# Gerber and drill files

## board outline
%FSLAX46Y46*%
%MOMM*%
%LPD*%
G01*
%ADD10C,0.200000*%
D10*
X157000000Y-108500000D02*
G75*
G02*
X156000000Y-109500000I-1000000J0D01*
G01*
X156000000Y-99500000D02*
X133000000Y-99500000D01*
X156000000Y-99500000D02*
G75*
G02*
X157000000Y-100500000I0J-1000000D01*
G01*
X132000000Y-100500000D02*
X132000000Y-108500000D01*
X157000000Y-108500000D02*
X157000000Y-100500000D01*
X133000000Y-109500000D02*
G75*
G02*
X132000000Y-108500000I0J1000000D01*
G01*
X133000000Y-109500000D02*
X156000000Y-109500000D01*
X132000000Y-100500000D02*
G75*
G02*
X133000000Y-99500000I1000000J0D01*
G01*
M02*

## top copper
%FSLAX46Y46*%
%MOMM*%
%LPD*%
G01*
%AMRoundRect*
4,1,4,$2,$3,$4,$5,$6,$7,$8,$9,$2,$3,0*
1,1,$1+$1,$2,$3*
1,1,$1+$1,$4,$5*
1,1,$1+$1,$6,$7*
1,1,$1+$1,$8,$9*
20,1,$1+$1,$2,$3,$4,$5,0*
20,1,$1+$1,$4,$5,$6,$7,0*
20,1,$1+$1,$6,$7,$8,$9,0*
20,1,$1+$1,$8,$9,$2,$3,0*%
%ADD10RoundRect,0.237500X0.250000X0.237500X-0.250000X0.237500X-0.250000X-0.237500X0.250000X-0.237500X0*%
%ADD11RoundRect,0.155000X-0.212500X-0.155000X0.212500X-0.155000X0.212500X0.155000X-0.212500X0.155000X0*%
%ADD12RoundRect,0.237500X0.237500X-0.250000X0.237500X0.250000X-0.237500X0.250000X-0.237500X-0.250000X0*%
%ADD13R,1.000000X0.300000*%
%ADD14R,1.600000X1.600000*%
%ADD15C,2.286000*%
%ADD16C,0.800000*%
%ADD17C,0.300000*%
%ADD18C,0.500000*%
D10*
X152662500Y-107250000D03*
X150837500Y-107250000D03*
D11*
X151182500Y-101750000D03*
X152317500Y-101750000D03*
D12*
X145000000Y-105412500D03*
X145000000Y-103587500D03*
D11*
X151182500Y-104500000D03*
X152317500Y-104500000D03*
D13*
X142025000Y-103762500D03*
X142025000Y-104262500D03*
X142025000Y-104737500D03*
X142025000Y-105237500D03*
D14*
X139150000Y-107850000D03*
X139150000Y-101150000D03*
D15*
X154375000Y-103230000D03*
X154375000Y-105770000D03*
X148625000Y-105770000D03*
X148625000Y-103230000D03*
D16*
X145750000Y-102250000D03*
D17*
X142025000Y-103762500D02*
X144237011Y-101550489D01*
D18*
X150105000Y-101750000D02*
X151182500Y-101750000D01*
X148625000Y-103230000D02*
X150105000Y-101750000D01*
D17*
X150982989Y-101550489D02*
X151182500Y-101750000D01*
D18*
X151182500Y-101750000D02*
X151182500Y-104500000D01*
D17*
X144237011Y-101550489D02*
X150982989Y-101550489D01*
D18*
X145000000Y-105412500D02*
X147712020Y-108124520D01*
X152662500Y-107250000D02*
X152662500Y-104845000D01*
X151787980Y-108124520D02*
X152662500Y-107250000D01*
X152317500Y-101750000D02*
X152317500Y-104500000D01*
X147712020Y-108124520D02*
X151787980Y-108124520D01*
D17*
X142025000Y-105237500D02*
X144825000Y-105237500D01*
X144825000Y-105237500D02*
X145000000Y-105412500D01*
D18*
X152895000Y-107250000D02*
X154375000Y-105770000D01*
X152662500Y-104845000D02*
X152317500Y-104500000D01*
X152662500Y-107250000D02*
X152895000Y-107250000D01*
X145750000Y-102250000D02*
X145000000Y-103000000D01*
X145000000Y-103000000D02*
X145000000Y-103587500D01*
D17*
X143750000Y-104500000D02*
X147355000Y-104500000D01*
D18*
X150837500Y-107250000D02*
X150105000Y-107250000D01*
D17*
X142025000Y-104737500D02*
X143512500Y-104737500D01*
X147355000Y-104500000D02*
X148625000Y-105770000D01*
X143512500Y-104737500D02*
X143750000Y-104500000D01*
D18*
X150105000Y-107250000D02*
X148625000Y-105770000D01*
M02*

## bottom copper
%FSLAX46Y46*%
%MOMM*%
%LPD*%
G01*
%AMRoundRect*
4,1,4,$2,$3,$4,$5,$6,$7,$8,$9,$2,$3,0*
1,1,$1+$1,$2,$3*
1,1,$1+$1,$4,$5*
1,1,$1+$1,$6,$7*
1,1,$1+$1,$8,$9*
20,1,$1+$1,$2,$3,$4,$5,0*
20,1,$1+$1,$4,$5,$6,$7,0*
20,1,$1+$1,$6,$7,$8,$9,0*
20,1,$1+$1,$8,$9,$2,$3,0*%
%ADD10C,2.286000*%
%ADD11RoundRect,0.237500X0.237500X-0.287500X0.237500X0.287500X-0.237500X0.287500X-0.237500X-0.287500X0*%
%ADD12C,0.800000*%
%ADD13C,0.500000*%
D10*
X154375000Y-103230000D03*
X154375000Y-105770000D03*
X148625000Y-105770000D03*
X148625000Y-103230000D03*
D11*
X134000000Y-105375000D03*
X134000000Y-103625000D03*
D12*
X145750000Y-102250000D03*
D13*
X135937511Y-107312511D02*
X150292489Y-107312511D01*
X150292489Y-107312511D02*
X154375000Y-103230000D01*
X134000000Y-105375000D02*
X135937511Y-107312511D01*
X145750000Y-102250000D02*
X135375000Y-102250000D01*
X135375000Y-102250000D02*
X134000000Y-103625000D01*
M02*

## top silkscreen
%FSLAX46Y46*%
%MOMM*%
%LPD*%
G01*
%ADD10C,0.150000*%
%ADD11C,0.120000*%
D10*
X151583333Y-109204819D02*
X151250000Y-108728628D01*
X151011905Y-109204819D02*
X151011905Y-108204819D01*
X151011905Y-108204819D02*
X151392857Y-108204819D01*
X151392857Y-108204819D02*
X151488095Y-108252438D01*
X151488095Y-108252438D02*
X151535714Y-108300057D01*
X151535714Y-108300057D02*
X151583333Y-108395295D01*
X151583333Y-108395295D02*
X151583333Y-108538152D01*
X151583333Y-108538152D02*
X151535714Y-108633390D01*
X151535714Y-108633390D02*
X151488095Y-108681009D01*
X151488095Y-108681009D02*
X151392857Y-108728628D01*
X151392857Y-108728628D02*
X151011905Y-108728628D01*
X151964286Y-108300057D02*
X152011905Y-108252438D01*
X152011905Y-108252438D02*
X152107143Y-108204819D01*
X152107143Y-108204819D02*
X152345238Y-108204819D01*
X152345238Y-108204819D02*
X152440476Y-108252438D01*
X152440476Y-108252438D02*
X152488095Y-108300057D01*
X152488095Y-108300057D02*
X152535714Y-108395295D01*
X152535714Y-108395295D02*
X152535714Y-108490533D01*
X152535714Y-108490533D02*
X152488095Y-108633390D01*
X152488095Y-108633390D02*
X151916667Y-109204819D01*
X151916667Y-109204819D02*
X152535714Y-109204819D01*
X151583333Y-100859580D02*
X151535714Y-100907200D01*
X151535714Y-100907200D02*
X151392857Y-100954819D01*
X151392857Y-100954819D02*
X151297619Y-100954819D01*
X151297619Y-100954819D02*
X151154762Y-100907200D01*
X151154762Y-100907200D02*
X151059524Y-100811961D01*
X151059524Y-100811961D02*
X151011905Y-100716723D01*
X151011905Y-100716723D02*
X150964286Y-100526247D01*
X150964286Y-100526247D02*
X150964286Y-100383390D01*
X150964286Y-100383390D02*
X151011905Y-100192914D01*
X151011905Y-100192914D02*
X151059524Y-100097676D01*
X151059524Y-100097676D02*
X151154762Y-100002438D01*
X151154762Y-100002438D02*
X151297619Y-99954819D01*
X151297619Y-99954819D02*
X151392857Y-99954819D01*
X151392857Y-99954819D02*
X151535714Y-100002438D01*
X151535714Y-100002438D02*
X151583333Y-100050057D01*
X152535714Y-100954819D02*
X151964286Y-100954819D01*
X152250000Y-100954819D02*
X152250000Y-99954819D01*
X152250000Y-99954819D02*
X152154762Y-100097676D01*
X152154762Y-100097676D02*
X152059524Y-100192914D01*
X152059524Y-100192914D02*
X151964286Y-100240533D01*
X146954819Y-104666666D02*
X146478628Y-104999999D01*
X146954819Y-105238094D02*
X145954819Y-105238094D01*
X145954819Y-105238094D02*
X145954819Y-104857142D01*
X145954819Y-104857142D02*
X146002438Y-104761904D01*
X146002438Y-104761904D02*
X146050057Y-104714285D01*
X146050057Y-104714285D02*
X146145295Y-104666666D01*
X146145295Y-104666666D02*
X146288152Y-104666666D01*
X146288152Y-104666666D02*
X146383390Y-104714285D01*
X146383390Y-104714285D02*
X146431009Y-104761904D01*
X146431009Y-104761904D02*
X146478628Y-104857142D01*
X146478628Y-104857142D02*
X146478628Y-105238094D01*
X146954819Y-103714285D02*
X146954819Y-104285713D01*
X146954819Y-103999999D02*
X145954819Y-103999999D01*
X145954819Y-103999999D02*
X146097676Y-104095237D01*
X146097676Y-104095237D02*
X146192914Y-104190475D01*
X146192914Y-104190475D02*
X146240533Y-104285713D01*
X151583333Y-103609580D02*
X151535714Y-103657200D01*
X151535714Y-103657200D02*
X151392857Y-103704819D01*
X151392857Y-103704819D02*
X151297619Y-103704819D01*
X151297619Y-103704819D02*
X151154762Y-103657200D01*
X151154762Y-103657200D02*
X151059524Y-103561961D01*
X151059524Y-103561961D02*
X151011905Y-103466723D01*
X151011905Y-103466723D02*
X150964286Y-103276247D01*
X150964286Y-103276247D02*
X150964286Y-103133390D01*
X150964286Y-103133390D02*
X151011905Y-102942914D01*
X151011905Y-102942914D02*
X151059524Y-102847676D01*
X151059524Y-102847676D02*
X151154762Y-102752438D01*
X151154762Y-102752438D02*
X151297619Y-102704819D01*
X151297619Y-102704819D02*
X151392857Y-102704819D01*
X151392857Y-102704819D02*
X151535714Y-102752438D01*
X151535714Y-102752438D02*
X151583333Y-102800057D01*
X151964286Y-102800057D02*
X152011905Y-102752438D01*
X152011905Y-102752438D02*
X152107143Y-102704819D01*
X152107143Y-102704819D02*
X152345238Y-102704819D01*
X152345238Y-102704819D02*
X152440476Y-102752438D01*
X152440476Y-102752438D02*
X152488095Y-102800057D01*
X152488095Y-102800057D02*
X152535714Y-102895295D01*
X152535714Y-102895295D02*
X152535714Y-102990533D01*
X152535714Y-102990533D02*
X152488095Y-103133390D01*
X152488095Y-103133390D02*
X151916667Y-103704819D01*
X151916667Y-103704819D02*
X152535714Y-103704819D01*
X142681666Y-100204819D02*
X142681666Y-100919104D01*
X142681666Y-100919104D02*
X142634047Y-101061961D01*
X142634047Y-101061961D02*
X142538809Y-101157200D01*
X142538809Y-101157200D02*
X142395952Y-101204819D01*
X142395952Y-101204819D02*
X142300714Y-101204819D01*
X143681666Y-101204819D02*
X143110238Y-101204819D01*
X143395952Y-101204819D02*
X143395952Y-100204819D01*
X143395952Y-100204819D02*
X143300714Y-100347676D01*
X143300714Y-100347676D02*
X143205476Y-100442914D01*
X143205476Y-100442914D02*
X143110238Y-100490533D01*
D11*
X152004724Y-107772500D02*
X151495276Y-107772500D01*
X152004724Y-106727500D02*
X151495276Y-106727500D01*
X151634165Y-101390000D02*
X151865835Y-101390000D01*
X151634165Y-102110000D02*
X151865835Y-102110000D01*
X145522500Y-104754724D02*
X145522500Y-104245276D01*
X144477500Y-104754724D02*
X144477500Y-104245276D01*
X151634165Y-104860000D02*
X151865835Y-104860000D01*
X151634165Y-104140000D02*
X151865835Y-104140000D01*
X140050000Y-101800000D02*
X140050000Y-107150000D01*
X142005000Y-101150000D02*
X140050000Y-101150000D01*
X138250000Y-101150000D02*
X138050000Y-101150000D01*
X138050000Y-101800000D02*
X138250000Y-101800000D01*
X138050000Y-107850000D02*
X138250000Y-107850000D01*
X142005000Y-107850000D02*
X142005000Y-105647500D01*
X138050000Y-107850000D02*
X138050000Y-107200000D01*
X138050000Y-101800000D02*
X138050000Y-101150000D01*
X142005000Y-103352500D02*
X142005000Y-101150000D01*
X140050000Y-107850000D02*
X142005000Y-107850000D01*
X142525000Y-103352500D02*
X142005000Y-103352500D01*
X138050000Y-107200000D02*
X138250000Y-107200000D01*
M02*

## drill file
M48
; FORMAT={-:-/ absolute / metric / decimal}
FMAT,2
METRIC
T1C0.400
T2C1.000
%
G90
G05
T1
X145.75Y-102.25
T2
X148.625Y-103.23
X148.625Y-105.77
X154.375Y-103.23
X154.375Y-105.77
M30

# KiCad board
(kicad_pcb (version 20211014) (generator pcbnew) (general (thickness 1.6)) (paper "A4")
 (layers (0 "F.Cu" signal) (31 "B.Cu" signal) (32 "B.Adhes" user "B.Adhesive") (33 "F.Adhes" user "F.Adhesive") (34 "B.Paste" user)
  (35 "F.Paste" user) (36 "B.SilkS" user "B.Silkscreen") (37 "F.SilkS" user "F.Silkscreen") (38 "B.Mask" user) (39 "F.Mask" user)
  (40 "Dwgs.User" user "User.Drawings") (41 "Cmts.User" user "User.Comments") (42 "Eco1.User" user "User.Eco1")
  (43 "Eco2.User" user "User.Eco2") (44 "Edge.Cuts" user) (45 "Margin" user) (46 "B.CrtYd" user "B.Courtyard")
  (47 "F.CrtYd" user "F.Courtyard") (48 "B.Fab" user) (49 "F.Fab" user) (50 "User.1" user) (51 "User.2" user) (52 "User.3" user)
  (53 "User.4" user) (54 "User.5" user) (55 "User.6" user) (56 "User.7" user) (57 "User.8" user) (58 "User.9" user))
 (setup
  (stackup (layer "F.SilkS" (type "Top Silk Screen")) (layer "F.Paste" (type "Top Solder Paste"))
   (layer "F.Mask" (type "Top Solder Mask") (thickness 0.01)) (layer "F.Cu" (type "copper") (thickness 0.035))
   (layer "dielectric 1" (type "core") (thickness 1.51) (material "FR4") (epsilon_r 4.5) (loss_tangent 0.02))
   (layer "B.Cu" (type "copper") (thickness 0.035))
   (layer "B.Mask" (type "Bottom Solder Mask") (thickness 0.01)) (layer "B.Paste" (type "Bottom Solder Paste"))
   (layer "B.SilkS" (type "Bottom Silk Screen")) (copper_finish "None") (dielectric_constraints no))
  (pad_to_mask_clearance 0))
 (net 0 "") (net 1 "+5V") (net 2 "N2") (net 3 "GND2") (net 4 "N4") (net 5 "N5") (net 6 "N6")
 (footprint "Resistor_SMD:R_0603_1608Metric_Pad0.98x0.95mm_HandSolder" (layer "F.Cu") (at 151.75 107.25 180)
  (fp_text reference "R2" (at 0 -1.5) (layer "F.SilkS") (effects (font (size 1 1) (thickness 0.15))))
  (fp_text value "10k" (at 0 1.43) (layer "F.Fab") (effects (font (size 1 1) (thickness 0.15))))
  (fp_line (start -0.254724 -0.5225) (end 0.254724 -0.5225) (layer "F.SilkS") (width 0.12))
  (fp_line (start -0.254724 0.5225) (end 0.254724 0.5225) (layer "F.SilkS") (width 0.12))
  (pad "1" smd roundrect (at -0.9125 0 180) (size 0.975 0.95) (layers "F.Cu" "F.Paste" "F.Mask") (roundrect_rratio 0.25) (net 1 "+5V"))
  (pad "2" smd roundrect (at 0.9125 0 180) (size 0.975 0.95) (layers "F.Cu" "F.Paste" "F.Mask") (roundrect_rratio 0.25) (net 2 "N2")))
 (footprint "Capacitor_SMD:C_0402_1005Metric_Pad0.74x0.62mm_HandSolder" (layer "F.Cu") (at 151.75 101.75)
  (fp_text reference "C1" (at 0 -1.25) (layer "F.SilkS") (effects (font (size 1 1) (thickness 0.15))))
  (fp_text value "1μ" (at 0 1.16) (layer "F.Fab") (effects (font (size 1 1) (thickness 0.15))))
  (fp_line (start -0.115835 -0.36) (end 0.115835 -0.36) (layer "F.SilkS") (width 0.12))
  (fp_line (start -0.115835 0.36) (end 0.115835 0.36) (layer "F.SilkS") (width 0.12))
  (pad "1" smd roundrect (at -0.5675 0) (size 0.735 0.62) (layers "F.Cu" "F.Paste" "F.Mask") (roundrect_rratio 0.25) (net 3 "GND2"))
  (pad "2" smd roundrect (at 0.5675 0) (size 0.735 0.62) (layers "F.Cu" "F.Paste" "F.Mask") (roundrect_rratio 0.25) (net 1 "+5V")))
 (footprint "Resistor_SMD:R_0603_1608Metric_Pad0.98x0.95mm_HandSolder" (layer "F.Cu") (at 145 104.5 90)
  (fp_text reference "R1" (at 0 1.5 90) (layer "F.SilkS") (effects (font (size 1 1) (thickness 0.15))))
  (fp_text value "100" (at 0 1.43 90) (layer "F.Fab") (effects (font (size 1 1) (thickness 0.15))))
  (fp_line (start -0.254724 0.5225) (end 0.254724 0.5225) (layer "F.SilkS") (width 0.12))
  (fp_line (start -0.254724 -0.5225) (end 0.254724 -0.5225) (layer "F.SilkS") (width 0.12))
  (pad "1" smd roundrect (at -0.9125 0 90) (size 0.975 0.95) (layers "F.Cu" "F.Paste" "F.Mask") (roundrect_rratio 0.25) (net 1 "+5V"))
  (pad "2" smd roundrect (at 0.9125 0 90) (size 0.975 0.95) (layers "F.Cu" "F.Paste" "F.Mask") (roundrect_rratio 0.25) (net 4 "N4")))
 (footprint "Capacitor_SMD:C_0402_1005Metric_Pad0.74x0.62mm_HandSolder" (layer "F.Cu") (at 151.75 104.5)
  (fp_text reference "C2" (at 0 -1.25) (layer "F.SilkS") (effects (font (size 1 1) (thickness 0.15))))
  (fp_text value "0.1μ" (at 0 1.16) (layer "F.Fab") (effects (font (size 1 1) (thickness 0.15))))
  (fp_line (start -0.115835 0.36) (end 0.115835 0.36) (layer "F.SilkS") (width 0.12))
  (fp_line (start -0.115835 -0.36) (end 0.115835 -0.36) (layer "F.SilkS") (width 0.12))
  (pad "1" smd roundrect (at -0.5675 0) (size 0.735 0.62) (layers "F.Cu" "F.Paste" "F.Mask") (roundrect_rratio 0.25) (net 3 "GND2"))
  (pad "2" smd roundrect (at 0.5675 0) (size 0.735 0.62) (layers "F.Cu" "F.Paste" "F.Mask") (roundrect_rratio 0.25) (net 1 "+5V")))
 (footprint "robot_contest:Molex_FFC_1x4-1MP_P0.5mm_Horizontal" (layer "F.Cu") (at 141 104.5 -90)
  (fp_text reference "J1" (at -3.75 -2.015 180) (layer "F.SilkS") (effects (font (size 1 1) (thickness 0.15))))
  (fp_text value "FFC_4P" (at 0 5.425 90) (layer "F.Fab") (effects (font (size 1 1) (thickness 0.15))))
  (fp_line (start -2.7 0.95) (end 2.65 0.95) (layer "F.SilkS") (width 0.12))
  (fp_line (start -3.35 -1.005) (end -3.35 0.95) (layer "F.SilkS") (width 0.12))
  (fp_line (start -3.35 2.75) (end -3.35 2.95) (layer "F.SilkS") (width 0.12))
  (fp_line (start -2.7 2.95) (end -2.7 2.75) (layer "F.SilkS") (width 0.12))
  (fp_line (start 3.35 2.95) (end 3.35 2.75) (layer "F.SilkS") (width 0.12))
  (fp_line (start 3.35 -1.005) (end 1.1475 -1.005) (layer "F.SilkS") (width 0.12))
  (fp_line (start 3.35 2.95) (end 2.7 2.95) (layer "F.SilkS") (width 0.12))
  (fp_line (start -2.7 2.95) (end -3.35 2.95) (layer "F.SilkS") (width 0.12))
  (fp_line (start -1.1475 -1.005) (end -3.35 -1.005) (layer "F.SilkS") (width 0.12))
  (fp_line (start 3.35 0.95) (end 3.35 -1.005) (layer "F.SilkS") (width 0.12))
  (fp_line (start -1.1475 -1.525) (end -1.1475 -1.005) (layer "F.SilkS") (width 0.12))
  (fp_line (start 2.7 2.95) (end 2.7 2.75) (layer "F.SilkS") (width 0.12))
  (pad "1" smd rect (at -0.7375 -1.025 270) (size 0.3 1) (layers "F.Cu" "F.Paste" "F.Mask") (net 3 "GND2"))
  (pad "2" smd rect (at -0.2375 -1.025 270) (size 0.3 1) (layers "F.Cu" "F.Paste" "F.Mask") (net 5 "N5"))
  (pad "3" smd rect (at 0.2375 -1.025 270) (size 0.3 1) (layers "F.Cu" "F.Paste" "F.Mask") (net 2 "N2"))
  (pad "4" smd rect (at 0.7375 -1.025 270) (size 0.3 1) (layers "F.Cu" "F.Paste" "F.Mask") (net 1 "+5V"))
  (pad "MP" smd rect (at 3.35 1.85 270) (size 1.6 1.6) (layers "F.Cu" "F.Paste" "F.Mask"))
  (pad "MP" smd rect (at -3.35 1.85 270) (size 1.6 1.6) (layers "F.Cu" "F.Paste" "F.Mask")))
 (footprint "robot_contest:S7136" (layer "B.Cu") (at 151.5 105.77 180)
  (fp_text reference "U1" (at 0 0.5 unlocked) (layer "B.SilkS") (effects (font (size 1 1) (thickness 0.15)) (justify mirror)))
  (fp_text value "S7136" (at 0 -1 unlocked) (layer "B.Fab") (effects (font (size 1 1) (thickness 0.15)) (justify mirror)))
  (pad "1" thru_hole circle (at -2.875 2.54 180) (size 2.286 2.286) (drill 1) (layers *.Cu *.Mask) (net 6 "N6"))
  (pad "2" thru_hole circle (at -2.875 0 180) (size 2.286 2.286) (drill 1) (layers *.Cu *.Mask) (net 1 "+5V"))
  (pad "3" thru_hole circle (at 2.875 0 180) (size 2.286 2.286) (drill 1) (layers *.Cu *.Mask) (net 2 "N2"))
  (pad "4" thru_hole circle (at 2.875 2.54 180) (size 2.286 2.286) (drill 1) (layers *.Cu *.Mask) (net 3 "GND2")))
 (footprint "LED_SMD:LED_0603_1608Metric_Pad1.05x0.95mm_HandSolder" (layer "B.Cu") (at 134 104.5 90)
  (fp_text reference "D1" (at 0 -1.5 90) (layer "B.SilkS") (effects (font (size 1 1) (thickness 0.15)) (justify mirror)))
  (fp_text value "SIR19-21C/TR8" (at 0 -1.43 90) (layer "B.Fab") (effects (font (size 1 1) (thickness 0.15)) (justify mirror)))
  (pad "1" smd roundrect (at -0.875 0 90) (size 1.05 0.95) (layers "B.Cu" "B.Paste" "B.Mask") (roundrect_rratio 0.25) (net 6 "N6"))
  (pad "2" smd roundrect (at 0.875 0 90) (size 1.05 0.95) (layers "B.Cu" "B.Paste" "B.Mask") (roundrect_rratio 0.25) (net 4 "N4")))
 (gr_arc (start 157 108.5) (mid 156.707107 109.207107) (end 156 109.5) (layer "Edge.Cuts") (width 0.2))
 (gr_line (start 156 99.5) (end 133 99.5) (layer "Edge.Cuts") (width 0.2))
 (gr_arc (start 156 99.5) (mid 156.707107 99.792893) (end 157 100.5) (layer "Edge.Cuts") (width 0.2))
 (gr_line (start 132 100.5) (end 132 108.5) (layer "Edge.Cuts") (width 0.2))
 (gr_line (start 157 108.5) (end 157 100.5) (layer "Edge.Cuts") (width 0.2))
 (gr_arc (start 133 109.5) (mid 132.292893 109.207107) (end 132 108.5) (layer "Edge.Cuts") (width 0.2))
 (gr_line (start 133 109.5) (end 156 109.5) (layer "Edge.Cuts") (width 0.2))
 (gr_arc (start 132 100.5) (mid 132.292893 99.792893) (end 133 99.5) (layer "Edge.Cuts") (width 0.2))
 (segment (start 142.025 103.7625) (end 144.237011 101.550489) (width 0.3) (layer "F.Cu") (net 3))
 (segment (start 150.105 101.75) (end 151.1825 101.75) (width 0.5) (layer "F.Cu") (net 3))
 (segment (start 148.625 103.23) (end 150.105 101.75) (width 0.5) (layer "F.Cu") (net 3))
 (segment (start 150.982989 101.550489) (end 151.1825 101.75) (width 0.3) (layer "F.Cu") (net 3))
 (segment (start 151.1825 101.75) (end 151.1825 104.5) (width 0.5) (layer "F.Cu") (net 3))
 (segment (start 144.237011 101.550489) (end 150.982989 101.550489) (width 0.3) (layer "F.Cu") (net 3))
 (segment (start 145 105.4125) (end 147.71202 108.12452) (width 0.5) (layer "F.Cu") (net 1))
 (segment (start 152.6625 107.25) (end 152.6625 104.845) (width 0.5) (layer "F.Cu") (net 1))
 (segment (start 151.78798 108.12452) (end 152.6625 107.25) (width 0.5) (layer "F.Cu") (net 1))
 (segment (start 152.3175 101.75) (end 152.3175 104.5) (width 0.5) (layer "F.Cu") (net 1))
 (segment (start 147.71202 108.12452) (end 151.78798 108.12452) (width 0.5) (layer "F.Cu") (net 1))
 (segment (start 142.025 105.2375) (end 144.825 105.2375) (width 0.3) (layer "F.Cu") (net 1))
 (segment (start 144.825 105.2375) (end 145 105.4125) (width 0.3) (layer "F.Cu") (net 1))
 (segment (start 152.895 107.25) (end 154.375 105.77) (width 0.5) (layer "F.Cu") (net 1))
 (segment (start 152.6625 104.845) (end 152.3175 104.5) (width 0.5) (layer "F.Cu") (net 1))
 (segment (start 152.6625 107.25) (end 152.895 107.25) (width 0.5) (layer "F.Cu") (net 1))
 (segment (start 135.937511 107.312511) (end 150.292489 107.312511) (width 0.5) (layer "B.Cu") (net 6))
 (segment (start 150.292489 107.312511) (end 154.375 103.23) (width 0.5) (layer "B.Cu") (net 6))
 (segment (start 134 105.375) (end 135.937511 107.312511) (width 0.5) (layer "B.Cu") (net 6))
 (segment (start 145.75 102.25) (end 145 103) (width 0.5) (layer "F.Cu") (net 4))
 (segment (start 145 103) (end 145 103.5875) (width 0.5) (layer "F.Cu") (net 4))
 (via (at 145.75 102.25) (size 0.8) (drill 0.4) (layers "F.Cu" "B.Cu") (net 4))
 (segment (start 145.75 102.25) (end 135.375 102.25) (width 0.5) (layer "B.Cu") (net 4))
 (segment (start 135.375 102.25) (end 134 103.625) (width 0.5) (layer "B.Cu") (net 4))
 (segment (start 143.75 104.5) (end 147.355 104.5) (width 0.3) (layer "F.Cu") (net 2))
 (segment (start 150.8375 107.25) (end 150.105 107.25) (width 0.5) (layer "F.Cu") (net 2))
 (segment (start 142.025 104.7375) (end 143.5125 104.7375) (width 0.3) (layer "F.Cu") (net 2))
 (segment (start 147.355 104.5) (end 148.625 105.77) (width 0.3) (layer "F.Cu") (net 2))
 (segment (start 143.5125 104.7375) (end 143.75 104.5) (width 0.3) (layer "F.Cu") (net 2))
 (segment (start 150.105 107.25) (end 148.625 105.77) (width 0.5) (layer "F.Cu") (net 2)))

